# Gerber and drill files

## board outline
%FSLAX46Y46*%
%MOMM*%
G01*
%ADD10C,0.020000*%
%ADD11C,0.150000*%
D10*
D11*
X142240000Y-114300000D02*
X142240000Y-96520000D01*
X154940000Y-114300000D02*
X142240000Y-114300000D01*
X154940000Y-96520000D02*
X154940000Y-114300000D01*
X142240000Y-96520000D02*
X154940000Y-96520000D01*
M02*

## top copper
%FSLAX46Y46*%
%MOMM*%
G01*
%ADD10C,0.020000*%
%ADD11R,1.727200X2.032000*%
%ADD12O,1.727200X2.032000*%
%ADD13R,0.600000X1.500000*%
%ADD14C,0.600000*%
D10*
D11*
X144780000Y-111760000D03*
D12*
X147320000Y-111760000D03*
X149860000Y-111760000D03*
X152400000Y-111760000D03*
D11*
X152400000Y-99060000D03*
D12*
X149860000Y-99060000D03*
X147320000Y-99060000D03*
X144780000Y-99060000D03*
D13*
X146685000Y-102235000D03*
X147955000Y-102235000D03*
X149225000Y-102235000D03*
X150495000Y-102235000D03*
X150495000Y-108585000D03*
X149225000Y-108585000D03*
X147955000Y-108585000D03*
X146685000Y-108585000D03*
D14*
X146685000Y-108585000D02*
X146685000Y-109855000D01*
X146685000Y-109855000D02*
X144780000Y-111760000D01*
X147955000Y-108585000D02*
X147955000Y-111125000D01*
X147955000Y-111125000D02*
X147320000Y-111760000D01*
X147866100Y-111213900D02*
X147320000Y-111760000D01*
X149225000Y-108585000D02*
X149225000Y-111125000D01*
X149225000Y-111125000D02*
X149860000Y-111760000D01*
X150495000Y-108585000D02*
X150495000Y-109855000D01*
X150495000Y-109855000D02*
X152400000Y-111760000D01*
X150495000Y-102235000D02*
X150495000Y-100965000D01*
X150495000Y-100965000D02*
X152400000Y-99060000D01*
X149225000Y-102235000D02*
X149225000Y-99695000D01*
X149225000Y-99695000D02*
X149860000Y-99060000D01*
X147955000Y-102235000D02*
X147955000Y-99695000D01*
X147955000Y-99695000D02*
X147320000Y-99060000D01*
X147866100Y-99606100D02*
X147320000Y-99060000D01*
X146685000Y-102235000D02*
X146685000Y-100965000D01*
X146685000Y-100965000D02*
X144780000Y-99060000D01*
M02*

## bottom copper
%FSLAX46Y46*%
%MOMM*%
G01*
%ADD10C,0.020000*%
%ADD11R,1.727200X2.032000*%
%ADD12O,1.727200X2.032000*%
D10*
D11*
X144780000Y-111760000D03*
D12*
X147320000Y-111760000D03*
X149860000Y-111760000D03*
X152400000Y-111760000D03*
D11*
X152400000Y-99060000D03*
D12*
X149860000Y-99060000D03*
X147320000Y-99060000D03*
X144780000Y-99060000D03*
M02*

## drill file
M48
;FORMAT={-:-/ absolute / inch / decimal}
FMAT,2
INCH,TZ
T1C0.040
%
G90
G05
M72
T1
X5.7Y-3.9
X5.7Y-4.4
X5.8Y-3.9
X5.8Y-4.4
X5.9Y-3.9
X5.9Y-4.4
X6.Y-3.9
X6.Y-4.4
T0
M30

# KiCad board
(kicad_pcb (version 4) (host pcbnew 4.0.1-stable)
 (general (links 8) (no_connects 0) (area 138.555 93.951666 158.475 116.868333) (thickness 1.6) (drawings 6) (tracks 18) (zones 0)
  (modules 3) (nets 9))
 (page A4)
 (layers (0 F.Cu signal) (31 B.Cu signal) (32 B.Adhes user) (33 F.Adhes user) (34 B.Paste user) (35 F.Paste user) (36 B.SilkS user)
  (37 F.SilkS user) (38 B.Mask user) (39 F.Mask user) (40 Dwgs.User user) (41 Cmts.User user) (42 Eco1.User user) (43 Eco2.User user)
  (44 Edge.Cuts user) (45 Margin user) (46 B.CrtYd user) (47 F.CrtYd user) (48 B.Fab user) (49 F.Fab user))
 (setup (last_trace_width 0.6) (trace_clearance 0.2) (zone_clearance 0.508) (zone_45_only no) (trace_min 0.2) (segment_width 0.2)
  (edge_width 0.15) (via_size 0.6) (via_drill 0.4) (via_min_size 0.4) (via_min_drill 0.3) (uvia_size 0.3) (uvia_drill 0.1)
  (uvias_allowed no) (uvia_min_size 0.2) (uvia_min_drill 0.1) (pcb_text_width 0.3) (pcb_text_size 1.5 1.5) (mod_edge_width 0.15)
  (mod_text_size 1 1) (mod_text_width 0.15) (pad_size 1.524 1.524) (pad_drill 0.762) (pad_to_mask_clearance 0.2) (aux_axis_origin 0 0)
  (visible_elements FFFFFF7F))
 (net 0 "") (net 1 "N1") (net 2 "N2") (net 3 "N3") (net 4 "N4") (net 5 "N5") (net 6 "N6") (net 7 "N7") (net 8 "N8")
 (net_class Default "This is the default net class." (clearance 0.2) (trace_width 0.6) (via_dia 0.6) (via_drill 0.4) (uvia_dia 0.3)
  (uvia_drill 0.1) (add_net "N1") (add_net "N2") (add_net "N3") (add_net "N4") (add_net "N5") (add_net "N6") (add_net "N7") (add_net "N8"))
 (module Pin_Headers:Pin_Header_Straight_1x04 (layer F.Cu) (at 144.78 111.76 90)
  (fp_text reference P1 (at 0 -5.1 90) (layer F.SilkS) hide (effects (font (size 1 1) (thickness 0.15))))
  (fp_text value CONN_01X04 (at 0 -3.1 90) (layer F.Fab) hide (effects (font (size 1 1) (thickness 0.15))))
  (pad 1 thru_hole rect (at 0 0 90) (size 2.032 1.7272) (drill 1.016) (layers *.Cu *.Mask F.SilkS) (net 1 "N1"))
  (pad 2 thru_hole oval (at 0 2.54 90) (size 2.032 1.7272) (drill 1.016) (layers *.Cu *.Mask F.SilkS) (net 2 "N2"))
  (pad 3 thru_hole oval (at 0 5.08 90) (size 2.032 1.7272) (drill 1.016) (layers *.Cu *.Mask F.SilkS) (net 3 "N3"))
  (pad 4 thru_hole oval (at 0 7.62 90) (size 2.032 1.7272) (drill 1.016) (layers *.Cu *.Mask F.SilkS) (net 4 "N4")))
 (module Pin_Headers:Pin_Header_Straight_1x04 (layer F.Cu) (at 152.4 99.06 270)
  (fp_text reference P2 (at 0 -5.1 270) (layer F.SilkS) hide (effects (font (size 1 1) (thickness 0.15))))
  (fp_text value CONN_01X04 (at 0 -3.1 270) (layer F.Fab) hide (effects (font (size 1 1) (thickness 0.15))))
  (pad 1 thru_hole rect (at 0 0 270) (size 2.032 1.7272) (drill 1.016) (layers *.Cu *.Mask F.SilkS) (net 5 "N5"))
  (pad 2 thru_hole oval (at 0 2.54 270) (size 2.032 1.7272) (drill 1.016) (layers *.Cu *.Mask F.SilkS) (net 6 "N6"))
  (pad 3 thru_hole oval (at 0 5.08 270) (size 2.032 1.7272) (drill 1.016) (layers *.Cu *.Mask F.SilkS) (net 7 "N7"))
  (pad 4 thru_hole oval (at 0 7.62 270) (size 2.032 1.7272) (drill 1.016) (layers *.Cu *.Mask F.SilkS) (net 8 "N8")))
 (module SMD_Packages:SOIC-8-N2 (layer F.Cu) (at 148.59 105.41)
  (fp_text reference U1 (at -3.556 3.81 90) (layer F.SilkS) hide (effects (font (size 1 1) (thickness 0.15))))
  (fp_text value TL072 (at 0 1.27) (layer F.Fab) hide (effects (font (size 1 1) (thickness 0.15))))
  (pad 8 smd rect (at -1.905 -3.175) (size 0.6 1.5) (layers F.Cu F.Paste F.Mask) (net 8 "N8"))
  (pad 7 smd rect (at -0.635 -3.175) (size 0.6 1.5) (layers F.Cu F.Paste F.Mask) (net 7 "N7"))
  (pad 6 smd rect (at 0.635 -3.175) (size 0.6 1.5) (layers F.Cu F.Paste F.Mask) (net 6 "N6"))
  (pad 5 smd rect (at 1.905 -3.175) (size 0.6 1.5) (layers F.Cu F.Paste F.Mask) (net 5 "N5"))
  (pad 4 smd rect (at 1.905 3.175) (size 0.6 1.5) (layers F.Cu F.Paste F.Mask) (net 4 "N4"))
  (pad 3 smd rect (at 0.635 3.175) (size 0.6 1.5) (layers F.Cu F.Paste F.Mask) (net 3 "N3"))
  (pad 2 smd rect (at -0.635 3.175) (size 0.6 1.5) (layers F.Cu F.Paste F.Mask) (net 2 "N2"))
  (pad 1 smd rect (at -1.905 3.175) (size 0.6 1.5) (layers F.Cu F.Paste F.Mask) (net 1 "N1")))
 (gr_line (start 142.24 114.3) (end 142.24 96.52) (angle 90) (layer Edge.Cuts) (width 0.15))
 (gr_line (start 154.94 114.3) (end 142.24 114.3) (angle 90) (layer Edge.Cuts) (width 0.15))
 (gr_line (start 154.94 96.52) (end 154.94 114.3) (angle 90) (layer Edge.Cuts) (width 0.15))
 (gr_line (start 142.24 96.52) (end 154.94 96.52) (angle 90) (layer Edge.Cuts) (width 0.15))
 (segment (start 146.685 108.585) (end 146.685 109.855) (width 0.6) (layer F.Cu) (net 1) (status 400000))
 (segment (start 146.685 109.855) (end 144.78 111.76) (width 0.6) (layer F.Cu) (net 1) (status 800000))
 (segment (start 147.955 108.585) (end 147.955 111.125) (width 0.6) (layer F.Cu) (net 2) (status C00000))
 (segment (start 147.955 111.125) (end 147.32 111.76) (width 0.6) (layer F.Cu) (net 2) (status C00000))
 (segment (start 147.8661 111.2139) (end 147.32 111.76) (width 0.6) (layer F.Cu) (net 2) (status C00000))
 (segment (start 149.225 108.585) (end 149.225 111.125) (width 0.6) (layer F.Cu) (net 3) (status C00000))
 (segment (start 149.225 111.125) (end 149.86 111.76) (width 0.6) (layer F.Cu) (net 3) (status C00000))
 (segment (start 150.495 108.585) (end 150.495 109.855) (width 0.6) (layer F.Cu) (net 4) (status 400000))
 (segment (start 150.495 109.855) (end 152.4 111.76) (width 0.6) (layer F.Cu) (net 4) (status 800000))
 (segment (start 150.495 102.235) (end 150.495 100.965) (width 0.6) (layer F.Cu) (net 5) (status 400000))
 (segment (start 150.495 100.965) (end 152.4 99.06) (width 0.6) (layer F.Cu) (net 5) (status 800000))
 (segment (start 149.225 102.235) (end 149.225 99.695) (width 0.6) (layer F.Cu) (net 6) (status C00000))
 (segment (start 149.225 99.695) (end 149.86 99.06) (width 0.6) (layer F.Cu) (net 6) (status C00000))
 (segment (start 147.955 102.235) (end 147.955 99.695) (width 0.6) (layer F.Cu) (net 7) (status C00000))
 (segment (start 147.955 99.695) (end 147.32 99.06) (width 0.6) (layer F.Cu) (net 7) (status C00000))
 (segment (start 147.8661 99.6061) (end 147.32 99.06) (width 0.6) (layer F.Cu) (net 7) (status C00000))
 (segment (start 146.685 102.235) (end 146.685 100.965) (width 0.6) (layer F.Cu) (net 8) (status 400000))
 (segment (start 146.685 100.965) (end 144.78 99.06) (width 0.6) (layer F.Cu) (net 8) (status 800000)))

